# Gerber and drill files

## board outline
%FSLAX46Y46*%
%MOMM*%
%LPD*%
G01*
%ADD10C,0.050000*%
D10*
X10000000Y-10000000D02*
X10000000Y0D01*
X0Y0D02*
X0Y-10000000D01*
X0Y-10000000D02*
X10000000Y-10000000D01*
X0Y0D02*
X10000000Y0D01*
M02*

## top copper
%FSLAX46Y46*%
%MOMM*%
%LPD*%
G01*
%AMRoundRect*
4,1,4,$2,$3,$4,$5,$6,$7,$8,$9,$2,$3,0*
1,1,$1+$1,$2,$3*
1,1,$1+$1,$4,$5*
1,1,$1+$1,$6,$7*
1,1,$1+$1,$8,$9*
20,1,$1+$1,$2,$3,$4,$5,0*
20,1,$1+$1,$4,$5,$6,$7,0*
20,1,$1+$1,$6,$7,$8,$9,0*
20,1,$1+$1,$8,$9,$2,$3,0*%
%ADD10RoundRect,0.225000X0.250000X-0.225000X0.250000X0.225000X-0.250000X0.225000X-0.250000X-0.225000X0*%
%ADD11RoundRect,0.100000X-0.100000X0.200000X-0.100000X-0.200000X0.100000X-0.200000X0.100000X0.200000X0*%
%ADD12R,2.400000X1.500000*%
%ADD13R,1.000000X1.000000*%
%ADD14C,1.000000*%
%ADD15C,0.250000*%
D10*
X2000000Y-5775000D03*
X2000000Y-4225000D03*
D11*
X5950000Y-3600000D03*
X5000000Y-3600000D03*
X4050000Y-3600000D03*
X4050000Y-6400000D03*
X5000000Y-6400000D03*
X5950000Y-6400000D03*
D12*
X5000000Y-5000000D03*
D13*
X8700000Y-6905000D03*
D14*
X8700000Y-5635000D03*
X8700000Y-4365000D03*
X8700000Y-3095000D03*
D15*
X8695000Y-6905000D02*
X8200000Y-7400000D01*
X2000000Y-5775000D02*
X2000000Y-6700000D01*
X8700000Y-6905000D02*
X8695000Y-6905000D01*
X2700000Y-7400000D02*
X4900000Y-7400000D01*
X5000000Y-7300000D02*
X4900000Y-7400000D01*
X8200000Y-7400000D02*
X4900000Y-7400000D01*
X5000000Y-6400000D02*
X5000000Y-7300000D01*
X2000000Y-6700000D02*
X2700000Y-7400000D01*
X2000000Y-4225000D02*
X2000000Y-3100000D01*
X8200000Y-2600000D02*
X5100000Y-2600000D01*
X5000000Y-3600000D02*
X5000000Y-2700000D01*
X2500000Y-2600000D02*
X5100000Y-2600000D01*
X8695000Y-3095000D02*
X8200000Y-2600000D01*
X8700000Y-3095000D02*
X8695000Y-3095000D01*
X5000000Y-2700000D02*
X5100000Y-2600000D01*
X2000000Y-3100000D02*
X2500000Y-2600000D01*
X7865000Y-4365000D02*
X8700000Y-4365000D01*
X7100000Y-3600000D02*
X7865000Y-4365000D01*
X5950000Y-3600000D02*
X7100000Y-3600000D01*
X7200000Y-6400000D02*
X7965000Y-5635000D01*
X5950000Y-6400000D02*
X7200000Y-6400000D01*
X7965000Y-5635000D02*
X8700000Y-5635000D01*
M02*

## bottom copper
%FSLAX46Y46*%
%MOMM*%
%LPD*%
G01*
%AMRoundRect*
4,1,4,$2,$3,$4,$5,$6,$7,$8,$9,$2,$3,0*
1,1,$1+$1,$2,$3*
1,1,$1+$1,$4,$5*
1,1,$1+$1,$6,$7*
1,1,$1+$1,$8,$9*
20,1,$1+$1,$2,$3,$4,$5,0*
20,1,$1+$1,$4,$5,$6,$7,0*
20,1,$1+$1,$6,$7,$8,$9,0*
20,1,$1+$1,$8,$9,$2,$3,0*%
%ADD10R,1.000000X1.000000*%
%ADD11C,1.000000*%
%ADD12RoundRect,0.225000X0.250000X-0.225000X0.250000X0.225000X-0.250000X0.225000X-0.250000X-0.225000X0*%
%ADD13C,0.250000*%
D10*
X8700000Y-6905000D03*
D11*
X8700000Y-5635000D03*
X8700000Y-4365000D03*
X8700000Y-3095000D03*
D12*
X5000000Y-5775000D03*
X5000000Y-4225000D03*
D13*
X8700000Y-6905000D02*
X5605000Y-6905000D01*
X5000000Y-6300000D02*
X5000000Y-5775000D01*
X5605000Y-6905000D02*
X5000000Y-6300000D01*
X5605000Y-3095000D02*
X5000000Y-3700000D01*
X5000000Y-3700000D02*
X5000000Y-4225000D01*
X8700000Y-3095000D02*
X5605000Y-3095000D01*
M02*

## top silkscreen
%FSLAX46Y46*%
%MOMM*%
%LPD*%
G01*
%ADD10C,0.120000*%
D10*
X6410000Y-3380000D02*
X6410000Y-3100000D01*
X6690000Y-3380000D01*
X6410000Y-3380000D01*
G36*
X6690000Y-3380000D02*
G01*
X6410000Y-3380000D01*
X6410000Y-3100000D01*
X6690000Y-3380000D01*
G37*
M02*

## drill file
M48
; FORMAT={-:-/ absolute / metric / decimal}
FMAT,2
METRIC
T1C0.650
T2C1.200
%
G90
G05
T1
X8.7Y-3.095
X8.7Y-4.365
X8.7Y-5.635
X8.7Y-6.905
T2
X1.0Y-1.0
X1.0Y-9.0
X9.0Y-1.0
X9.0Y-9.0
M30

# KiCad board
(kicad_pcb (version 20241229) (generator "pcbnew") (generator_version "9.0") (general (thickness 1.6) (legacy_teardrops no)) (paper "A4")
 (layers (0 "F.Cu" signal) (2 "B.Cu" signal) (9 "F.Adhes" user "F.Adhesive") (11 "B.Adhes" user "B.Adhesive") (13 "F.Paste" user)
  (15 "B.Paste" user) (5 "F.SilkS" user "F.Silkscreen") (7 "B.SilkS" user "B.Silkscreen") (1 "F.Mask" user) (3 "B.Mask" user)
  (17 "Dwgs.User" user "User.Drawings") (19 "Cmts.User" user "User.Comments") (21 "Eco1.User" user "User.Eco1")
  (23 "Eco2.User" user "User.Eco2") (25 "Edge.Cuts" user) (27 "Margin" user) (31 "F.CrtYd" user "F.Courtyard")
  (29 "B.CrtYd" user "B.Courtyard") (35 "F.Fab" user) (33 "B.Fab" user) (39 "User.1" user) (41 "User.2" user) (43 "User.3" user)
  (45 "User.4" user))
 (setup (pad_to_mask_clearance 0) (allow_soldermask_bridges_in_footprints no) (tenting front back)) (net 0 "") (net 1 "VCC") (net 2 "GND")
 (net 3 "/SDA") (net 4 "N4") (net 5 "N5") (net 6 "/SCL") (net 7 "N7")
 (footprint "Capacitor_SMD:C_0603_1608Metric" (layer "F.Cu") (at 2 5 90)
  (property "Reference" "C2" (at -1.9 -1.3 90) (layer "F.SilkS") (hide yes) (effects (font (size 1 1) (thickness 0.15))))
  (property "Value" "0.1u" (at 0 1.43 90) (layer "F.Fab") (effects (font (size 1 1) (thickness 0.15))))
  (pad "1" smd roundrect (at -0.775 0 90) (size 0.9 0.95) (layers "F.Cu" "F.Mask" "F.Paste") (roundrect_rratio 0.25) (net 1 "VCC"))
  (pad "2" smd roundrect (at 0.775 0 90) (size 0.9 0.95) (layers "F.Cu" "F.Mask" "F.Paste") (roundrect_rratio 0.25) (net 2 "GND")))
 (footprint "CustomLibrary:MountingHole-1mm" (layer "F.Cu") (at 1 1)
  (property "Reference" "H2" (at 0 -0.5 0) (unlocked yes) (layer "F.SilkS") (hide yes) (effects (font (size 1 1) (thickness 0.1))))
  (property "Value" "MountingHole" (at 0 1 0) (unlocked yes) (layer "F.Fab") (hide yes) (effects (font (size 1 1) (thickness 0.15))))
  (pad "" np_thru_hole circle (at 0 0) (size 1 1) (drill 1.2) (layers "*.Cu" "*.Mask")))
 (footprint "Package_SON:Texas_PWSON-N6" (layer "F.Cu") (at 5 5 -90)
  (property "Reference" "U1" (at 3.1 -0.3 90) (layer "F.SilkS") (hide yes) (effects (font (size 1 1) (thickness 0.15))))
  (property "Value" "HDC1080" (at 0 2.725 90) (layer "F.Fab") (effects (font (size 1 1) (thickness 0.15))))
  (fp_poly
   (pts (xy -1.62 -1.41) (xy -1.9 -1.41) (xy -1.62 -1.69) (xy -1.62 -1.41)) (stroke (width 0.12) (type solid)) (fill yes) (layer "F.SilkS"))
  (pad "" smd roundrect (at -0.4 -0.65 270) (size 0.6 1) (layers "F.Paste") (roundrect_rratio 0.25) (solder_paste_margin_ratio -0.2))
  (pad "" smd roundrect (at -0.4 0.65 270) (size 0.6 1) (layers "F.Paste") (roundrect_rratio 0.25) (solder_paste_margin_ratio -0.2))
  (pad "" smd roundrect (at 0.4 -0.65 270) (size 0.6 1) (layers "F.Paste") (roundrect_rratio 0.25) (solder_paste_margin_ratio -0.2))
  (pad "" smd roundrect (at 0.4 0.65 270) (size 0.6 1) (layers "F.Paste") (roundrect_rratio 0.25) (solder_paste_margin_ratio -0.2))
  (pad "1" smd roundrect (at -1.4 -0.95 270) (size 0.6 0.4) (layers "F.Cu" "F.Mask" "F.Paste") (roundrect_rratio 0.25) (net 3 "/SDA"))
  (pad "2" smd roundrect (at -1.4 0 270) (size 0.6 0.4) (layers "F.Cu" "F.Mask" "F.Paste") (roundrect_rratio 0.25) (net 2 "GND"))
  (pad "3" smd roundrect (at -1.4 0.95 270) (size 0.6 0.4) (layers "F.Cu" "F.Mask" "F.Paste") (roundrect_rratio 0.25) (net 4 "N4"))
  (pad "4" smd roundrect (at 1.4 0.95 270) (size 0.6 0.4) (layers "F.Cu" "F.Mask" "F.Paste") (roundrect_rratio 0.25) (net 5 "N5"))
  (pad "5" smd roundrect (at 1.4 0 270) (size 0.6 0.4) (layers "F.Cu" "F.Mask" "F.Paste") (roundrect_rratio 0.25) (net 1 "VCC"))
  (pad "6" smd roundrect (at 1.4 -0.95 270) (size 0.6 0.4) (layers "F.Cu" "F.Mask" "F.Paste") (roundrect_rratio 0.25) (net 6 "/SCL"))
  (pad "7" smd rect (at 0 0 270) (size 1.5 2.4) (layers "F.Cu" "F.Mask") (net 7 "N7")))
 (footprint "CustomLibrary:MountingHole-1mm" (layer "F.Cu") (at 9 0.9)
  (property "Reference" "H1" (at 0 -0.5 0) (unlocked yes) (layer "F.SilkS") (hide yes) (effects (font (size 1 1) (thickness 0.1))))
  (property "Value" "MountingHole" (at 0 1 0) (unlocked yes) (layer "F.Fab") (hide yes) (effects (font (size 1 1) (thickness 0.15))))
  (pad "" np_thru_hole circle (at 0 0.1) (size 1 1) (drill 1.2) (layers "*.Cu" "*.Mask")))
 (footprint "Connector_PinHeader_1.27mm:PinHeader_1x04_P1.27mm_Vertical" (layer "F.Cu") (at 8.7 6.905 180)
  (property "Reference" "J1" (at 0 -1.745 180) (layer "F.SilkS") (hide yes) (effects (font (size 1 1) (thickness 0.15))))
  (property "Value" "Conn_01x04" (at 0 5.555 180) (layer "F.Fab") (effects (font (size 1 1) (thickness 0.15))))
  (pad "1" thru_hole rect (at 0 0 180) (size 1 1) (drill 0.65) (layers "*.Cu" "*.Mask") (remove_unused_layers no) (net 1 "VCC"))
  (pad "2" thru_hole circle (at 0 1.27 180) (size 1 1) (drill 0.65) (layers "*.Cu" "*.Mask") (remove_unused_layers no) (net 6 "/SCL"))
  (pad "3" thru_hole circle (at 0 2.54 180) (size 1 1) (drill 0.65) (layers "*.Cu" "*.Mask") (remove_unused_layers no) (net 3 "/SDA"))
  (pad "4" thru_hole circle (at 0 3.81 180) (size 1 1) (drill 0.65) (layers "*.Cu" "*.Mask") (remove_unused_layers no) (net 2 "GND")))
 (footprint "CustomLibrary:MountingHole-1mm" (layer "F.Cu") (at 1 9)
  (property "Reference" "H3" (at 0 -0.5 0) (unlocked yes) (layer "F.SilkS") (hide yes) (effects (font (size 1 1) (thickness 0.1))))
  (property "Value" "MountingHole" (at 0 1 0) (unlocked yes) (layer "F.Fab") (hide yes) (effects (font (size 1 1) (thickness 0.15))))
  (pad "" np_thru_hole circle (at 0 0) (size 1 1) (drill 1.2) (layers "*.Cu" "*.Mask")))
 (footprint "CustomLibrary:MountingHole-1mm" (layer "F.Cu") (at 9 9)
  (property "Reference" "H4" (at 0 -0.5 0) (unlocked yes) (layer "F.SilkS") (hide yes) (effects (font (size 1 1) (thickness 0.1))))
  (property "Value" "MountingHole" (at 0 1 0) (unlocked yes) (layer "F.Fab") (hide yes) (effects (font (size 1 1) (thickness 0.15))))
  (pad "" np_thru_hole circle (at 0 0) (size 1 1) (drill 1.2) (layers "*.Cu" "*.Mask")))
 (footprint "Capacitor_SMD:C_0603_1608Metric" (layer "B.Cu") (at 5 5 90)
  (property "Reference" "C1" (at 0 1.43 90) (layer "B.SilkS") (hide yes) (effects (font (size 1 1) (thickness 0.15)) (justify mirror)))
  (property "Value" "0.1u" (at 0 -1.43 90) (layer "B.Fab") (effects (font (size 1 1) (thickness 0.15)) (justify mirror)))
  (pad "1" smd roundrect (at -0.775 0 90) (size 0.9 0.95) (layers "B.Cu" "B.Mask" "B.Paste") (roundrect_rratio 0.25) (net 1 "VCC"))
  (pad "2" smd roundrect (at 0.775 0 90) (size 0.9 0.95) (layers "B.Cu" "B.Mask" "B.Paste") (roundrect_rratio 0.25) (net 2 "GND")))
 (gr_line (start 10 10) (end 10 0) (stroke (width 0.05) (type default)) (layer "Edge.Cuts"))
 (gr_line (start 0 0) (end 0 10) (stroke (width 0.05) (type solid)) (layer "Edge.Cuts"))
 (gr_line (start 0 10) (end 10 10) (stroke (width 0.05) (type solid)) (layer "Edge.Cuts"))
 (gr_line (start 0 0) (end 10 0) (stroke (width 0.05) (type solid)) (layer "Edge.Cuts"))
 (segment (start 8.695 6.905) (end 8.2 7.4) (width 0.25) (layer "F.Cu") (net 1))
 (segment (start 2 5.775) (end 2 6.7) (width 0.25) (layer "F.Cu") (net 1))
 (segment (start 8.7 6.905) (end 8.695 6.905) (width 0.25) (layer "F.Cu") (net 1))
 (segment (start 2.7 7.4) (end 4.9 7.4) (width 0.25) (layer "F.Cu") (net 1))
 (segment (start 5 7.3) (end 4.9 7.4) (width 0.25) (layer "F.Cu") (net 1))
 (segment (start 8.2 7.4) (end 4.9 7.4) (width 0.25) (layer "F.Cu") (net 1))
 (segment (start 5 6.4) (end 5 7.3) (width 0.25) (layer "F.Cu") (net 1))
 (segment (start 2 6.7) (end 2.7 7.4) (width 0.25) (layer "F.Cu") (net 1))
 (segment (start 8.7 6.905) (end 5.605 6.905) (width 0.25) (layer "B.Cu") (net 1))
 (segment (start 5 6.3) (end 5 5.775) (width 0.25) (layer "B.Cu") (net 1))
 (segment (start 5.605 6.905) (end 5 6.3) (width 0.25) (layer "B.Cu") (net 1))
 (segment (start 2 4.225) (end 2 3.1) (width 0.25) (layer "F.Cu") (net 2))
 (segment (start 8.2 2.6) (end 5.1 2.6) (width 0.25) (layer "F.Cu") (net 2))
 (segment (start 5 3.6) (end 5 2.7) (width 0.25) (layer "F.Cu") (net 2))
 (segment (start 2.5 2.6) (end 5.1 2.6) (width 0.25) (layer "F.Cu") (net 2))
 (segment (start 8.695 3.095) (end 8.2 2.6) (width 0.25) (layer "F.Cu") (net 2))
 (segment (start 8.7 3.095) (end 8.695 3.095) (width 0.25) (layer "F.Cu") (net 2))
 (segment (start 5 2.7) (end 5.1 2.6) (width 0.25) (layer "F.Cu") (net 2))
 (segment (start 2 3.1) (end 2.5 2.6) (width 0.25) (layer "F.Cu") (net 2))
 (segment (start 5.605 3.095) (end 5 3.7) (width 0.25) (layer "B.Cu") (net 2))
 (segment (start 5 3.7) (end 5 4.225) (width 0.25) (layer "B.Cu") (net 2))
 (segment (start 8.7 3.095) (end 5.605 3.095) (width 0.25) (layer "B.Cu") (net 2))
 (segment (start 7.865 4.365) (end 8.7 4.365) (width 0.25) (layer "F.Cu") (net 3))
 (segment (start 7.1 3.6) (end 7.865 4.365) (width 0.25) (layer "F.Cu") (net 3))
 (segment (start 5.95 3.6) (end 7.1 3.6) (width 0.25) (layer "F.Cu") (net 3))
 (segment (start 7.2 6.4) (end 7.965 5.635) (width 0.25) (layer "F.Cu") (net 6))
 (segment (start 5.95 6.4) (end 7.2 6.4) (width 0.25) (layer "F.Cu") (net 6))
 (segment (start 7.965 5.635) (end 8.7 5.635) (width 0.25) (layer "F.Cu") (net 6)))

